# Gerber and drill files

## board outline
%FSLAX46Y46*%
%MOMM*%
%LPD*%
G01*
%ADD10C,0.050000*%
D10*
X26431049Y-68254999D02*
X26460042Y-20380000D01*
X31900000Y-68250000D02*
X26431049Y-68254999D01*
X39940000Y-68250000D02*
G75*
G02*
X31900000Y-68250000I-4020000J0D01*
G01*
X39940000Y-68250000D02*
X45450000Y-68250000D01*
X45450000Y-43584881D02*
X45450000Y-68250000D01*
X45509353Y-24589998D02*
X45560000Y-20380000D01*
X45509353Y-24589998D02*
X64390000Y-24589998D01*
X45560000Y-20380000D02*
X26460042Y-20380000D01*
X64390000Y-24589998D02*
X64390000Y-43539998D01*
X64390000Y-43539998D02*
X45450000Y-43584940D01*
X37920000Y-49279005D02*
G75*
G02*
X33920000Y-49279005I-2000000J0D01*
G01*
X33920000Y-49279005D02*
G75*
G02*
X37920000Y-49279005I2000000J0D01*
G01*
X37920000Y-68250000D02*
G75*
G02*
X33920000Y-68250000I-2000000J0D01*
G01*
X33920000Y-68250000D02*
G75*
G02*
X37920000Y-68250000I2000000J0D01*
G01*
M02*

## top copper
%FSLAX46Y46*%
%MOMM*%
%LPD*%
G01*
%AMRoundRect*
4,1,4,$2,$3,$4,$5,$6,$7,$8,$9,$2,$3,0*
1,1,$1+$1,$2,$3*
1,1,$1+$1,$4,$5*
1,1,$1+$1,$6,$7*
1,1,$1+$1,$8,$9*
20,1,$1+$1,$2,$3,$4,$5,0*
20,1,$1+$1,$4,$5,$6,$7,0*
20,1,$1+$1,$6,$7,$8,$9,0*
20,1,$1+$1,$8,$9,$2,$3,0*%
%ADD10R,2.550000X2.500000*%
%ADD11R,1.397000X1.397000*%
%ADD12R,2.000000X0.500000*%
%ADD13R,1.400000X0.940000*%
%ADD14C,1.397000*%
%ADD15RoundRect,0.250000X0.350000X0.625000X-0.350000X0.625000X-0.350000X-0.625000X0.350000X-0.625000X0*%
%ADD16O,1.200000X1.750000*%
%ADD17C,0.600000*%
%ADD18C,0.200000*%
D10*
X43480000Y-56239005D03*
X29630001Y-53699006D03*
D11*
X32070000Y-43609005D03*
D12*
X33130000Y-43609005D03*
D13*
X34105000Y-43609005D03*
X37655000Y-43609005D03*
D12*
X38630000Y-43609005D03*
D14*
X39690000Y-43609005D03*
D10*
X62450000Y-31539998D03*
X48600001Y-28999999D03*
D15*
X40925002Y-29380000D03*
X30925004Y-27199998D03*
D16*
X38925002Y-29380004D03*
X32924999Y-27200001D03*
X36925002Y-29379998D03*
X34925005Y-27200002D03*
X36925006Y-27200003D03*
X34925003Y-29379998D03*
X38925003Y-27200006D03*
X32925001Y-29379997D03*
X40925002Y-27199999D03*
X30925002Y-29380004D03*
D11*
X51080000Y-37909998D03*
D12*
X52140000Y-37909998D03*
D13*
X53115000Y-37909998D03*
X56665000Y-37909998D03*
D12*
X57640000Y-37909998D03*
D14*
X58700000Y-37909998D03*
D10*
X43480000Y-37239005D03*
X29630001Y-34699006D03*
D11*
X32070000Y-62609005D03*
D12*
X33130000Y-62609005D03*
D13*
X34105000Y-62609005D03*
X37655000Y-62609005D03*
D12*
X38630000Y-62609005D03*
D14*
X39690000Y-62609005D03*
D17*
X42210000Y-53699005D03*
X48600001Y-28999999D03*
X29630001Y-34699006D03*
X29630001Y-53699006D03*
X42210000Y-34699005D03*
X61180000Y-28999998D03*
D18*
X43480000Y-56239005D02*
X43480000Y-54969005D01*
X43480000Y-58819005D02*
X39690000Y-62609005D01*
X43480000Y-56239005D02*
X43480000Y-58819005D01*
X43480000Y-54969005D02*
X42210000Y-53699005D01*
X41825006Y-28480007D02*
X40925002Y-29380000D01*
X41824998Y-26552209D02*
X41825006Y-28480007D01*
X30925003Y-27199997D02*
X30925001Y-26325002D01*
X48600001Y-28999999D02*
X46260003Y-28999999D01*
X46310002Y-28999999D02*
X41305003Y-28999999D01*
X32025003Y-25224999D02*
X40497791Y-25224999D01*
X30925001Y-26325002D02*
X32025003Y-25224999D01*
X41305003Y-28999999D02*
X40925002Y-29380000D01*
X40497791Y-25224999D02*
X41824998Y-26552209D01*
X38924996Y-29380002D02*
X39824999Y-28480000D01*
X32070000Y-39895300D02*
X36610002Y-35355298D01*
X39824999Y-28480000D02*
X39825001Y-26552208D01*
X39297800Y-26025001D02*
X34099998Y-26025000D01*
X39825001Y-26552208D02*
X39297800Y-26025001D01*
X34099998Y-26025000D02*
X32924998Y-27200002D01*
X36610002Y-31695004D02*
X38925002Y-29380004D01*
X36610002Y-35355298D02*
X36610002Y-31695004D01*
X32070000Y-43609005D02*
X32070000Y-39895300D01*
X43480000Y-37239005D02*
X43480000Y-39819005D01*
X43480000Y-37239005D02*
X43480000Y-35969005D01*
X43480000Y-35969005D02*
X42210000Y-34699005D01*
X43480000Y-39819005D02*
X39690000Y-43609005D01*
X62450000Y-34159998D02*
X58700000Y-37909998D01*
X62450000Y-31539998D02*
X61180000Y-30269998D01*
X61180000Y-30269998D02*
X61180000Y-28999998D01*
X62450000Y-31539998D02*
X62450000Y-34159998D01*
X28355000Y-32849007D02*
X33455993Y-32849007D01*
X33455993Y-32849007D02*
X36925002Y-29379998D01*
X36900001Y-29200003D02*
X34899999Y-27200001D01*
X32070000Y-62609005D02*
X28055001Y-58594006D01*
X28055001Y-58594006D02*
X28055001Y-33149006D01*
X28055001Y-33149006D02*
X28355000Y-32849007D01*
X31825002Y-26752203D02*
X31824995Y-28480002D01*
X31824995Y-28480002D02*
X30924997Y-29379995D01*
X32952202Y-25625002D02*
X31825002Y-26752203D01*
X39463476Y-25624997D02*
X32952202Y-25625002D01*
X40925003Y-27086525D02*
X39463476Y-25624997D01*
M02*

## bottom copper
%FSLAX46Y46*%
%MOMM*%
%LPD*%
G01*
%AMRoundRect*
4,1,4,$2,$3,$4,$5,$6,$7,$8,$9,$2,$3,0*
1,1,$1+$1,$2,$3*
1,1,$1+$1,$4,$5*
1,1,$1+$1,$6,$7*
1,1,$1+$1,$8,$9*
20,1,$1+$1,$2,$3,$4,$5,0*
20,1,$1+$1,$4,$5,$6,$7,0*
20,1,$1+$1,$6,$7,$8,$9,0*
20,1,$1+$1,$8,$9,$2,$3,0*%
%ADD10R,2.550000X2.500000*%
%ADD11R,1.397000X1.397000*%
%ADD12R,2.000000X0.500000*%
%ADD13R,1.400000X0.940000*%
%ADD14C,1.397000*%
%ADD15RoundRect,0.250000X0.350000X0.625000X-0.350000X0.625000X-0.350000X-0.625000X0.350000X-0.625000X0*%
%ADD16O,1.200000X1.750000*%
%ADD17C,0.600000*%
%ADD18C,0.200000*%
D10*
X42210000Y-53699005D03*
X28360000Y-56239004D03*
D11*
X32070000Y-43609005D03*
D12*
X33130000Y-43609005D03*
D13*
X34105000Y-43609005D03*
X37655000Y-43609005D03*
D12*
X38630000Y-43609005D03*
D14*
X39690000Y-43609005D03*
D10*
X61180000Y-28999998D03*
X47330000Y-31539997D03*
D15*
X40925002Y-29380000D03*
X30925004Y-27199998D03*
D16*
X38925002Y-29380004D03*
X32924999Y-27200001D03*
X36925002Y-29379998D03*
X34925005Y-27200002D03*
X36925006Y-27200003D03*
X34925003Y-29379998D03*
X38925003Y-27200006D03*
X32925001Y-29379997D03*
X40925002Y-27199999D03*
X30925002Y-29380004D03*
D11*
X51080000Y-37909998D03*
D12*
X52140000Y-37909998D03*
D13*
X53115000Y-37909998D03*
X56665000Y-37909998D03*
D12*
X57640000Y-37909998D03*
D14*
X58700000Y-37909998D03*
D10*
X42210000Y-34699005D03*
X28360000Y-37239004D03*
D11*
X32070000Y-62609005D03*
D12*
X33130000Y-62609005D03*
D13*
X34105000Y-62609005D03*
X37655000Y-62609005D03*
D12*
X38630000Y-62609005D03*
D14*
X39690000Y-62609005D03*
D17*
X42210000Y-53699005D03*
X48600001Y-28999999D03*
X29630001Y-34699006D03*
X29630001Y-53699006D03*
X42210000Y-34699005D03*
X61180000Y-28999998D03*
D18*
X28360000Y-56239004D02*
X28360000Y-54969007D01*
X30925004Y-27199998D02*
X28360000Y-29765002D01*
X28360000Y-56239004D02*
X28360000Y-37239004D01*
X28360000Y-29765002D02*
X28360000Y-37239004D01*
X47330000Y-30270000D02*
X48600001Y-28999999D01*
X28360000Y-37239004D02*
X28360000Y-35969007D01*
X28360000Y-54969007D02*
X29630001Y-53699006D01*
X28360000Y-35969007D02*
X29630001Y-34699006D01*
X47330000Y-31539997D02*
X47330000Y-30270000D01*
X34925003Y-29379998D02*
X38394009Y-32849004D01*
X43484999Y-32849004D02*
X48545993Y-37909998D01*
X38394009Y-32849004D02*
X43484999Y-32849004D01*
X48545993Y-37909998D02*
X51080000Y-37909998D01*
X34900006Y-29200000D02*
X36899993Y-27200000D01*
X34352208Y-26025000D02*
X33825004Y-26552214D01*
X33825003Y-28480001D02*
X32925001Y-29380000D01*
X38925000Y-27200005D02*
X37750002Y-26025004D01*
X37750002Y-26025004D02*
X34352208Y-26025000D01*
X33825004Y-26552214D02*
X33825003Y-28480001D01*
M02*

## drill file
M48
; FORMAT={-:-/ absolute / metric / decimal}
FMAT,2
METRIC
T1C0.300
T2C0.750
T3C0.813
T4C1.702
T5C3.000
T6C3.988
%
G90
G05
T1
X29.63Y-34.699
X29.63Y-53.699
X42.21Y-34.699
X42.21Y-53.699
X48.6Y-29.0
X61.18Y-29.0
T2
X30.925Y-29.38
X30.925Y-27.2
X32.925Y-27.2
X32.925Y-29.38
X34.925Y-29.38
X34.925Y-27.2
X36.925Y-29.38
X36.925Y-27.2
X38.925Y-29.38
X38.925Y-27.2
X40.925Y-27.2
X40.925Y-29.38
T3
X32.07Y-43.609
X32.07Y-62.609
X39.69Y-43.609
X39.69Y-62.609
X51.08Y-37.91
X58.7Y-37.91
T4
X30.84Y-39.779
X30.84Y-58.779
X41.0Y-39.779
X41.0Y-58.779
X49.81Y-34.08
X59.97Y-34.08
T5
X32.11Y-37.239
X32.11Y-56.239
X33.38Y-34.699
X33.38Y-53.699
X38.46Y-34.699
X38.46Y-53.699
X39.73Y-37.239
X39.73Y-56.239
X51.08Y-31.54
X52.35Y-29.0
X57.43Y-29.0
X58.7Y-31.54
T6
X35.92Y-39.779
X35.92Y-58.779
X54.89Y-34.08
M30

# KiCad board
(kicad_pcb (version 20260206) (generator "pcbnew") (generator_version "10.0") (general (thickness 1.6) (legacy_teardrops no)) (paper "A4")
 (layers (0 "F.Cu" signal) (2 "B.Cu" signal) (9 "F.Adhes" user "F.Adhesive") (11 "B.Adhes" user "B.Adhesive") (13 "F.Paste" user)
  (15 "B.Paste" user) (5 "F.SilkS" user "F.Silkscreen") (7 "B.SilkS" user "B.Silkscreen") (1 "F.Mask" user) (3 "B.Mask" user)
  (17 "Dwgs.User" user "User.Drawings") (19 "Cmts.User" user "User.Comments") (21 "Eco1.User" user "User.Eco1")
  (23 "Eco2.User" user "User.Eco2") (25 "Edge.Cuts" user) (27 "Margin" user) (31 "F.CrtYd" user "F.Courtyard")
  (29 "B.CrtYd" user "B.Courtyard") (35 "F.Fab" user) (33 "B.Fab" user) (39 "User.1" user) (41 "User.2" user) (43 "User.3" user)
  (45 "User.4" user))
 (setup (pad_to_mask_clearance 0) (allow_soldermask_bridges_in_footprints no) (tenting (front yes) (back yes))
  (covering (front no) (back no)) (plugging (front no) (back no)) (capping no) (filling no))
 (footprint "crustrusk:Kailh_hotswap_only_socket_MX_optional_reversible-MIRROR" (layer "F.Cu") (at 35.92 58.779005)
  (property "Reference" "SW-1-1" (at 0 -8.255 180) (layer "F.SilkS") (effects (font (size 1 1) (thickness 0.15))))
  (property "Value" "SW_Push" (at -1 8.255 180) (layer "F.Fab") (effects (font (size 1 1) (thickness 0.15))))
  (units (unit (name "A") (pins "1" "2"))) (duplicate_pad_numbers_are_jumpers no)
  (pad "" np_thru_hole circle (at -5.08 0) (size 1.7018 1.7018) (drill 1.7018) (layers "*.Cu" "*.Mask"))
  (pad "" np_thru_hole circle (at -3.81 -2.54 180) (size 3 3) (drill 3) (layers "*.Cu" "*.Mask"))
  (pad "" np_thru_hole circle (at -2.54 -5.079998) (size 3 3) (drill 3) (layers "*.Cu" "*.Mask"))
  (pad "" np_thru_hole circle (at 0 0) (size 3.9878 3.9878) (drill 3.9878) (layers "*.Cu" "*.Mask"))
  (pad "" np_thru_hole circle (at 2.540002 -5.080001 180) (size 3 3) (drill 3) (layers "*.Cu" "*.Mask"))
  (pad "" np_thru_hole circle (at 3.81 -2.54) (size 3 3) (drill 3) (layers "*.Cu" "*.Mask"))
  (pad "" np_thru_hole circle (at 5.08 0) (size 1.7018 1.7018) (drill 1.7018) (layers "*.Cu" "*.Mask"))
  (pad "1" smd rect (at 6.29 -5.08 180) (size 2.55 2.5) (layers "B.Cu" "B.Mask" "B.Paste") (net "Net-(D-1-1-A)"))
  (pad "1" smd rect (at 7.56 -2.54) (size 2.55 2.5) (layers "F.Cu" "F.Mask" "F.Paste") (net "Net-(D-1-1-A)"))
  (pad "2" smd rect (at -7.56 -2.540001 180) (size 2.55 2.5) (layers "B.Cu" "B.Mask" "B.Paste") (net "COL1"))
  (pad "2" smd rect (at -6.289999 -5.079999) (size 2.55 2.5) (layers "F.Cu" "F.Mask" "F.Paste") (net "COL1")))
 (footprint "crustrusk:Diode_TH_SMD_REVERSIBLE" (layer "F.Cu") (at 35.88 43.609005)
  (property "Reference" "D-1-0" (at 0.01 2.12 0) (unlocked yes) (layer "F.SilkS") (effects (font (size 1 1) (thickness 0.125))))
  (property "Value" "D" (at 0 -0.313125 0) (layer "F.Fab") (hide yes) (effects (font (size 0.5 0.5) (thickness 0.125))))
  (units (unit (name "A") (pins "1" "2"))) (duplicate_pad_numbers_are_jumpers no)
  (pad "1" thru_hole rect (at -3.81 0) (size 1.397 1.397) (drill 0.8128) (layers "*.Cu" "*.Mask") (remove_unused_layers no) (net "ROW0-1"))
  (pad "1" smd rect (at -2.75 0 180) (size 2 0.5) (layers "F.Cu") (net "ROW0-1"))
  (pad "1" smd rect (at -2.75 0) (size 2 0.5) (layers "B.Cu") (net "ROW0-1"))
  (pad "1" smd rect (at -1.775 0 180) (size 1.4 0.94) (layers "F.Cu" "F.Mask" "F.Paste") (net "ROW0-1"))
  (pad "1" smd rect (at -1.775 0) (size 1.4 0.94) (layers "B.Cu" "B.Mask" "B.Paste") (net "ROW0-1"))
  (pad "2" smd rect (at 1.775 0 180) (size 1.4 0.94) (layers "F.Cu" "F.Mask" "F.Paste") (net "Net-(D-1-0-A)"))
  (pad "2" smd rect (at 1.775 0) (size 1.4 0.94) (layers "B.Cu" "B.Mask" "B.Paste") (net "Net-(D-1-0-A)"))
  (pad "2" smd rect (at 2.75 0 180) (size 2 0.5) (layers "F.Cu") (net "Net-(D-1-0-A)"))
  (pad "2" smd rect (at 2.75 0) (size 2 0.5) (layers "B.Cu") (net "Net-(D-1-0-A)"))
  (pad "2" thru_hole circle (at 3.81 0) (size 1.397 1.397) (drill 0.8128) (layers "*.Cu" "*.Mask") (remove_unused_layers no)
   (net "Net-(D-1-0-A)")))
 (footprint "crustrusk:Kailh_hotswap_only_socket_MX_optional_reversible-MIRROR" (layer "F.Cu") (at 54.89 34.079998)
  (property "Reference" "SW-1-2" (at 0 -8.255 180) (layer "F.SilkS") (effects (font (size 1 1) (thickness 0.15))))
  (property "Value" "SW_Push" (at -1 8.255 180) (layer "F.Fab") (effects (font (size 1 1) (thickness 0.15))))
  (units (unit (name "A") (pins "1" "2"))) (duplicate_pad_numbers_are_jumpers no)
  (pad "" np_thru_hole circle (at -5.08 0) (size 1.7018 1.7018) (drill 1.7018) (layers "*.Cu" "*.Mask"))
  (pad "" np_thru_hole circle (at -3.81 -2.54 180) (size 3 3) (drill 3) (layers "*.Cu" "*.Mask"))
  (pad "" np_thru_hole circle (at -2.54 -5.079998) (size 3 3) (drill 3) (layers "*.Cu" "*.Mask"))
  (pad "" np_thru_hole circle (at 0 0) (size 3.9878 3.9878) (drill 3.9878) (layers "*.Cu" "*.Mask"))
  (pad "" np_thru_hole circle (at 2.540002 -5.080001 180) (size 3 3) (drill 3) (layers "*.Cu" "*.Mask"))
  (pad "" np_thru_hole circle (at 3.81 -2.54) (size 3 3) (drill 3) (layers "*.Cu" "*.Mask"))
  (pad "" np_thru_hole circle (at 5.08 0) (size 1.7018 1.7018) (drill 1.7018) (layers "*.Cu" "*.Mask"))
  (pad "1" smd rect (at 6.29 -5.08 180) (size 2.55 2.5) (layers "B.Cu" "B.Mask" "B.Paste") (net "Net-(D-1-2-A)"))
  (pad "1" smd rect (at 7.56 -2.54) (size 2.55 2.5) (layers "F.Cu" "F.Mask" "F.Paste") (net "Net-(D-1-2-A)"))
  (pad "2" smd rect (at -7.56 -2.540001 180) (size 2.55 2.5) (layers "B.Cu" "B.Mask" "B.Paste") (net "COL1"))
  (pad "2" smd rect (at -6.289999 -5.079999) (size 2.55 2.5) (layers "F.Cu" "F.Mask" "F.Paste") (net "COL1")))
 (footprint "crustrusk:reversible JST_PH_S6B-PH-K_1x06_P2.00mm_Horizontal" (layer "F.Cu") (at 40.925002 29.38 180)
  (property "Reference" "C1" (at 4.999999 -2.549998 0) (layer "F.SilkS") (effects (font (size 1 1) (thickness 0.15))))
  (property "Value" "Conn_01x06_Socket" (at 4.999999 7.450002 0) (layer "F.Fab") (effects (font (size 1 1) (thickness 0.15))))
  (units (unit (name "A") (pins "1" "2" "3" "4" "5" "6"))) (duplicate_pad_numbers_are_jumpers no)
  (pad "1" thru_hole roundrect (at 0 0 180) (size 1.2 1.75) (drill 0.75) (layers "*.Cu" "*.Mask") (remove_unused_layers no)
   (roundrect_rratio 0.208333) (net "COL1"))
  (pad "1" thru_hole roundrect (at 9.999998 2.180002 180) (size 1.2 1.75) (drill 0.75) (layers "*.Cu" "*.Mask") (remove_unused_layers no)
   (roundrect_rratio 0.208333) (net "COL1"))
  (pad "2" thru_hole oval (at 2 -0.000004 180) (size 1.2 1.75) (drill 0.75) (layers "*.Cu" "*.Mask") (remove_unused_layers no)
   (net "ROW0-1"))
  (pad "2" thru_hole oval (at 8.000003 2.179999 180) (size 1.2 1.75) (drill 0.75) (layers "*.Cu" "*.Mask") (remove_unused_layers no)
   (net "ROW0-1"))
  (pad "3" thru_hole oval (at 4 0.000002 180) (size 1.2 1.75) (drill 0.75) (layers "*.Cu" "*.Mask") (remove_unused_layers no) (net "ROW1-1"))
  (pad "3" thru_hole oval (at 5.999997 2.179998 180) (size 1.2 1.75) (drill 0.75) (layers "*.Cu" "*.Mask") (remove_unused_layers no)
   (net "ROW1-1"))
  (pad "4" thru_hole oval (at 3.999996 2.179997 180) (size 1.2 1.75) (drill 0.75) (layers "*.Cu" "*.Mask") (remove_unused_layers no)
   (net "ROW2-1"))
  (pad "4" thru_hole oval (at 5.999999 0.000002 180) (size 1.2 1.75) (drill 0.75) (layers "*.Cu" "*.Mask") (remove_unused_layers no)
   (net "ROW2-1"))
  (pad "5" thru_hole oval (at 1.999999 2.179994 180) (size 1.2 1.75) (drill 0.75) (layers "*.Cu" "*.Mask") (remove_unused_layers no)
   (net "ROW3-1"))
  (pad "5" thru_hole oval (at 8.000001 0.000003 180) (size 1.2 1.75) (drill 0.75) (layers "*.Cu" "*.Mask") (remove_unused_layers no)
   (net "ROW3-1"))
  (pad "6" thru_hole oval (at 0 2.180001 180) (size 1.2 1.75) (drill 0.75) (layers "*.Cu" "*.Mask") (remove_unused_layers no) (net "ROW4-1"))
  (pad "6" thru_hole oval (at 10 -0.000004 180) (size 1.2 1.75) (drill 0.75) (layers "*.Cu" "*.Mask") (remove_unused_layers no)
   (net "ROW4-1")))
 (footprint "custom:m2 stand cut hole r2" (layer "F.Cu") (at 35.92 49.279005)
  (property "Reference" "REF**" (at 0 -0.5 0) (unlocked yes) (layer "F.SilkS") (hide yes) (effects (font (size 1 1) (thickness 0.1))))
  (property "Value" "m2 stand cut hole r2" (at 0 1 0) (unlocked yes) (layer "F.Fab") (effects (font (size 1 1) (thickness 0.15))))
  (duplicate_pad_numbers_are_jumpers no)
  (fp_circle (center 0 0) (end 2 0) (stroke (width 0.05) (type default)) (fill no) (layer "Edge.Cuts")))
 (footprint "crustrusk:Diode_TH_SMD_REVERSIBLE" (layer "F.Cu") (at 54.89 37.909998)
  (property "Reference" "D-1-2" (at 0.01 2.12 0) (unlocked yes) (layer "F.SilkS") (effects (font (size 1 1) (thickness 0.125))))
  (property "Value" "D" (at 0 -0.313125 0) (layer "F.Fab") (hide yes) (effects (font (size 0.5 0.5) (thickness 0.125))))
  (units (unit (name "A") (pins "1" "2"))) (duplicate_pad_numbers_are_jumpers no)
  (pad "1" thru_hole rect (at -3.81 0) (size 1.397 1.397) (drill 0.8128) (layers "*.Cu" "*.Mask") (remove_unused_layers no) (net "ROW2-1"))
  (pad "1" smd rect (at -2.75 0 180) (size 2 0.5) (layers "F.Cu") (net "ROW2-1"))
  (pad "1" smd rect (at -2.75 0) (size 2 0.5) (layers "B.Cu") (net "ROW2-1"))
  (pad "1" smd rect (at -1.775 0 180) (size 1.4 0.94) (layers "F.Cu" "F.Mask" "F.Paste") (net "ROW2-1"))
  (pad "1" smd rect (at -1.775 0) (size 1.4 0.94) (layers "B.Cu" "B.Mask" "B.Paste") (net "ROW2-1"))
  (pad "2" smd rect (at 1.775 0 180) (size 1.4 0.94) (layers "F.Cu" "F.Mask" "F.Paste") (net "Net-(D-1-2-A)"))
  (pad "2" smd rect (at 1.775 0) (size 1.4 0.94) (layers "B.Cu" "B.Mask" "B.Paste") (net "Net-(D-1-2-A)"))
  (pad "2" smd rect (at 2.75 0 180) (size 2 0.5) (layers "F.Cu") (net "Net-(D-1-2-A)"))
  (pad "2" smd rect (at 2.75 0) (size 2 0.5) (layers "B.Cu") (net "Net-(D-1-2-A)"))
  (pad "2" thru_hole circle (at 3.81 0) (size 1.397 1.397) (drill 0.8128) (layers "*.Cu" "*.Mask") (remove_unused_layers no)
   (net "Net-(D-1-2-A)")))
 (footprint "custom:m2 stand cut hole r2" (layer "F.Cu") (at 35.92 68.25)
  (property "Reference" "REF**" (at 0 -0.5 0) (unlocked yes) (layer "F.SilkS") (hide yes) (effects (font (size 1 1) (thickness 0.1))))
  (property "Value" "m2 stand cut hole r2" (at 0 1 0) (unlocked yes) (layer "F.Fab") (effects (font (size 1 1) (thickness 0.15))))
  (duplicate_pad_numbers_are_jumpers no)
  (fp_circle (center 0 0) (end 2 0) (stroke (width 0.05) (type default)) (fill no) (layer "Edge.Cuts")))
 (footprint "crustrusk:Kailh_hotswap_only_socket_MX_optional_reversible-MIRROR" (layer "F.Cu") (at 35.92 39.779005)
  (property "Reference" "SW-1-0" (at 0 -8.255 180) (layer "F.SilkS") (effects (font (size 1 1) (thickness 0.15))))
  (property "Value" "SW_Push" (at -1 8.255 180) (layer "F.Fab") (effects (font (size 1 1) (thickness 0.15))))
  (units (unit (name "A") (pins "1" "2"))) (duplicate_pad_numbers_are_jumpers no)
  (pad "" np_thru_hole circle (at -5.08 0) (size 1.7018 1.7018) (drill 1.7018) (layers "*.Cu" "*.Mask"))
  (pad "" np_thru_hole circle (at -3.81 -2.54 180) (size 3 3) (drill 3) (layers "*.Cu" "*.Mask"))
  (pad "" np_thru_hole circle (at -2.54 -5.079998) (size 3 3) (drill 3) (layers "*.Cu" "*.Mask"))
  (pad "" np_thru_hole circle (at 0 0) (size 3.9878 3.9878) (drill 3.9878) (layers "*.Cu" "*.Mask"))
  (pad "" np_thru_hole circle (at 2.540002 -5.080001 180) (size 3 3) (drill 3) (layers "*.Cu" "*.Mask"))
  (pad "" np_thru_hole circle (at 3.81 -2.54) (size 3 3) (drill 3) (layers "*.Cu" "*.Mask"))
  (pad "" np_thru_hole circle (at 5.08 0) (size 1.7018 1.7018) (drill 1.7018) (layers "*.Cu" "*.Mask"))
  (pad "1" smd rect (at 6.29 -5.08 180) (size 2.55 2.5) (layers "B.Cu" "B.Mask" "B.Paste") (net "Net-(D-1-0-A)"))
  (pad "1" smd rect (at 7.56 -2.54) (size 2.55 2.5) (layers "F.Cu" "F.Mask" "F.Paste") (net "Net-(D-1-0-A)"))
  (pad "2" smd rect (at -7.56 -2.540001 180) (size 2.55 2.5) (layers "B.Cu" "B.Mask" "B.Paste") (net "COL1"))
  (pad "2" smd rect (at -6.289999 -5.079999) (size 2.55 2.5) (layers "F.Cu" "F.Mask" "F.Paste") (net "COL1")))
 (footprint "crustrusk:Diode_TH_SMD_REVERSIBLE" (layer "F.Cu") (at 35.88 62.609005)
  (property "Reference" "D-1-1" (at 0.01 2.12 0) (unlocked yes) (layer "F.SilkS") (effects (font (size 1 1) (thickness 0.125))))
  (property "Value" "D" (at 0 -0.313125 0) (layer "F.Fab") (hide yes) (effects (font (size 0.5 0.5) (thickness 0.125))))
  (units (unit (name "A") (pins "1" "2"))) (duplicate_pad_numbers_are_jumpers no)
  (pad "1" thru_hole rect (at -3.81 0) (size 1.397 1.397) (drill 0.8128) (layers "*.Cu" "*.Mask") (remove_unused_layers no) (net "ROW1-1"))
  (pad "1" smd rect (at -2.75 0 180) (size 2 0.5) (layers "F.Cu") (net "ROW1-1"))
  (pad "1" smd rect (at -2.75 0) (size 2 0.5) (layers "B.Cu") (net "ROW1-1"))
  (pad "1" smd rect (at -1.775 0 180) (size 1.4 0.94) (layers "F.Cu" "F.Mask" "F.Paste") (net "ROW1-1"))
  (pad "1" smd rect (at -1.775 0) (size 1.4 0.94) (layers "B.Cu" "B.Mask" "B.Paste") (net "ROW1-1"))
  (pad "2" smd rect (at 1.775 0 180) (size 1.4 0.94) (layers "F.Cu" "F.Mask" "F.Paste") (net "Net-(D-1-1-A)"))
  (pad "2" smd rect (at 1.775 0) (size 1.4 0.94) (layers "B.Cu" "B.Mask" "B.Paste") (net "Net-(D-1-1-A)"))
  (pad "2" smd rect (at 2.75 0 180) (size 2 0.5) (layers "F.Cu") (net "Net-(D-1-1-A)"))
  (pad "2" smd rect (at 2.75 0) (size 2 0.5) (layers "B.Cu") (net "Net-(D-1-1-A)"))
  (pad "2" thru_hole circle (at 3.81 0) (size 1.397 1.397) (drill 0.8128) (layers "*.Cu" "*.Mask") (remove_unused_layers no)
   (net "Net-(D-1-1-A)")))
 (gr_line (start 26.431049 68.254999) (end 26.460042 20.38) (stroke (width 0.05) (type default)) (layer "Edge.Cuts"))
 (gr_line (start 31.9 68.25) (end 26.431049 68.254999) (stroke (width 0.05) (type default)) (layer "Edge.Cuts"))
 (gr_arc (start 39.94 68.25) (mid 35.92 72.27) (end 31.9 68.25) (stroke (width 0.05) (type default)) (layer "Edge.Cuts"))
 (gr_line (start 39.94 68.25) (end 45.45 68.25) (stroke (width 0.05) (type default)) (layer "Edge.Cuts"))
 (gr_line (start 45.45 43.584881) (end 45.45 68.25) (stroke (width 0.05) (type default)) (layer "Edge.Cuts"))
 (gr_line (start 45.509353 24.589998) (end 45.56 20.38) (stroke (width 0.05) (type default)) (layer "Edge.Cuts"))
 (gr_line (start 45.509353 24.589998) (end 64.39 24.589998) (stroke (width 0.05) (type default)) (layer "Edge.Cuts"))
 (gr_line (start 45.56 20.38) (end 26.460042 20.38) (stroke (width 0.05) (type default)) (layer "Edge.Cuts"))
 (gr_line (start 64.39 24.589998) (end 64.39 43.539998) (stroke (width 0.05) (type default)) (layer "Edge.Cuts"))
 (gr_line (start 64.39 43.539998) (end 45.45 43.58494) (stroke (width 0.05) (type default)) (layer "Edge.Cuts"))
 (segment (start 43.48 56.239005) (end 43.48 54.969005) (width 0.2) (layer "F.Cu") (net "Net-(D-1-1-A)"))
 (segment (start 43.48 58.819005) (end 39.69 62.609005) (width 0.2) (layer "F.Cu") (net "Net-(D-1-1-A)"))
 (segment (start 43.48 56.239005) (end 43.48 58.819005) (width 0.2) (layer "F.Cu") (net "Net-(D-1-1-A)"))
 (segment (start 43.48 54.969005) (end 42.21 53.699005) (width 0.2) (layer "F.Cu") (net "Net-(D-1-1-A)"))
 (via (at 42.21 53.699005) (size 0.6) (drill 0.3) (layers "F.Cu" "B.Cu") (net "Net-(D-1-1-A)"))
 (segment (start 41.825006 28.480007) (end 40.925002 29.38) (width 0.2) (layer "F.Cu") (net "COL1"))
 (segment (start 41.824998 26.552209) (end 41.825006 28.480007) (width 0.2) (layer "F.Cu") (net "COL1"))
 (segment (start 30.925003 27.199997) (end 30.925001 26.325002) (width 0.2) (layer "F.Cu") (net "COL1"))
 (segment (start 48.600001 28.999999) (end 46.260003 28.999999) (width 0.2) (layer "F.Cu") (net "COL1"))
 (segment (start 46.310002 28.999999) (end 41.305003 28.999999) (width 0.2) (layer "F.Cu") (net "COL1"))
 (segment (start 32.025003 25.224999) (end 40.497791 25.224999) (width 0.2) (layer "F.Cu") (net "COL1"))
 (segment (start 30.925001 26.325002) (end 32.025003 25.224999) (width 0.2) (layer "F.Cu") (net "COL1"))
 (segment (start 41.305003 28.999999) (end 40.925002 29.38) (width 0.2) (layer "F.Cu") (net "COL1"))
 (segment (start 40.497791 25.224999) (end 41.824998 26.552209) (width 0.2) (layer "F.Cu") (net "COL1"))
 (via (at 48.600001 28.999999) (size 0.6) (drill 0.3) (layers "F.Cu" "B.Cu") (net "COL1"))
 (via (at 29.630001 34.699006) (size 0.6) (drill 0.3) (layers "F.Cu" "B.Cu") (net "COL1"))
 (via (at 29.630001 53.699006) (size 0.6) (drill 0.3) (layers "F.Cu" "B.Cu") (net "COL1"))
 (segment (start 28.36 56.239004) (end 28.36 54.969007) (width 0.2) (layer "B.Cu") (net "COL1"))
 (segment (start 30.925004 27.199998) (end 28.36 29.765002) (width 0.2) (layer "B.Cu") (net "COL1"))
 (segment (start 28.36 56.239004) (end 28.36 37.239004) (width 0.2) (layer "B.Cu") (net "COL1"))
 (segment (start 28.36 29.765002) (end 28.36 37.239004) (width 0.2) (layer "B.Cu") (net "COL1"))
 (segment (start 47.33 30.27) (end 48.600001 28.999999) (width 0.2) (layer "B.Cu") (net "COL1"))
 (segment (start 28.36 37.239004) (end 28.36 35.969007) (width 0.2) (layer "B.Cu") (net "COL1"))
 (segment (start 28.36 54.969007) (end 29.630001 53.699006) (width 0.2) (layer "B.Cu") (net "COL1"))
 (segment (start 28.36 35.969007) (end 29.630001 34.699006) (width 0.2) (layer "B.Cu") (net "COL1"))
 (segment (start 47.33 31.539997) (end 47.33 30.27) (width 0.2) (layer "B.Cu") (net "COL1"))
 (segment (start 38.924996 29.380002) (end 39.824999 28.48) (width 0.2) (layer "F.Cu") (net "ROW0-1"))
 (segment (start 32.07 39.8953) (end 36.610002 35.355298) (width 0.2) (layer "F.Cu") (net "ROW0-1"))
 (segment (start 39.824999 28.48) (end 39.825001 26.552208) (width 0.2) (layer "F.Cu") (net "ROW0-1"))
 (segment (start 39.2978 26.025001) (end 34.099998 26.025) (width 0.2) (layer "F.Cu") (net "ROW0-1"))
 (segment (start 39.825001 26.552208) (end 39.2978 26.025001) (width 0.2) (layer "F.Cu") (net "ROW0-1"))
 (segment (start 34.099998 26.025) (end 32.924998 27.200002) (width 0.2) (layer "F.Cu") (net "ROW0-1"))
 (segment (start 36.610002 31.695004) (end 38.925002 29.380004) (width 0.2) (layer "F.Cu") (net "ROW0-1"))
 (segment (start 36.610002 35.355298) (end 36.610002 31.695004) (width 0.2) (layer "F.Cu") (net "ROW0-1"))
 (segment (start 32.07 43.609005) (end 32.07 39.8953) (width 0.2) (layer "F.Cu") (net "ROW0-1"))
 (segment (start 43.48 37.239005) (end 43.48 39.819005) (width 0.2) (layer "F.Cu") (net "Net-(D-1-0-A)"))
 (segment (start 43.48 37.239005) (end 43.48 35.969005) (width 0.2) (layer "F.Cu") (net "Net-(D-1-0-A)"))
 (segment (start 43.48 35.969005) (end 42.21 34.699005) (width 0.2) (layer "F.Cu") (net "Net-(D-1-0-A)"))
 (segment (start 43.48 39.819005) (end 39.69 43.609005) (width 0.2) (layer "F.Cu") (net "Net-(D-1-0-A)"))
 (via (at 42.21 34.699005) (size 0.6) (drill 0.3) (layers "F.Cu" "B.Cu") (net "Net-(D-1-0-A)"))
 (segment (start 62.45 34.159998) (end 58.7 37.909998) (width 0.2) (layer "F.Cu") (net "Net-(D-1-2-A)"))
 (segment (start 62.45 31.539998) (end 61.18 30.269998) (width 0.2) (layer "F.Cu") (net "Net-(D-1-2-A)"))
 (segment (start 61.18 30.269998) (end 61.18 28.999998) (width 0.2) (layer "F.Cu") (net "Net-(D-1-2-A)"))
 (segment (start 62.45 31.539998) (end 62.45 34.159998) (width 0.2) (layer "F.Cu") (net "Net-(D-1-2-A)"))
 (via (at 61.18 28.999998) (size 0.6) (drill 0.3) (layers "F.Cu" "B.Cu") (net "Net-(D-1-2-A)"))
 (segment (start 28.355 32.849007) (end 33.455993 32.849007) (width 0.2) (layer "F.Cu") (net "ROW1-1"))
 (segment (start 33.455993 32.849007) (end 36.925002 29.379998) (width 0.2) (layer "F.Cu") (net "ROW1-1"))
 (segment (start 36.900001 29.200003) (end 34.899999 27.200001) (width 0.2) (layer "F.Cu") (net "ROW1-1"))
 (segment (start 32.07 62.609005) (end 28.055001 58.594006) (width 0.2) (layer "F.Cu") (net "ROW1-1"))
 (segment (start 28.055001 58.594006) (end 28.055001 33.149006) (width 0.2) (layer "F.Cu") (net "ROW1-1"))
 (segment (start 28.055001 33.149006) (end 28.355 32.849007) (width 0.2) (layer "F.Cu") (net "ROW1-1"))
 (segment (start 34.925003 29.379998) (end 38.394009 32.849004) (width 0.2) (layer "B.Cu") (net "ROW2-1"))
 (segment (start 43.484999 32.849004) (end 48.545993 37.909998) (width 0.2) (layer "B.Cu") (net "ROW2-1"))
 (segment (start 38.394009 32.849004) (end 43.484999 32.849004) (width 0.2) (layer "B.Cu") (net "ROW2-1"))
 (segment (start 48.545993 37.909998) (end 51.08 37.909998) (width 0.2) (layer "B.Cu") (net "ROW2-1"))
 (segment (start 34.900006 29.2) (end 36.899993 27.2) (width 0.2) (layer "B.Cu") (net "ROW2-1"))
 (segment (start 34.352208 26.025) (end 33.825004 26.552214) (width 0.2) (layer "B.Cu") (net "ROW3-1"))
 (segment (start 33.825003 28.480001) (end 32.925001 29.38) (width 0.2) (layer "B.Cu") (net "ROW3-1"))
 (segment (start 38.925 27.200005) (end 37.750002 26.025004) (width 0.2) (layer "B.Cu") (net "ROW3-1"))
 (segment (start 37.750002 26.025004) (end 34.352208 26.025) (width 0.2) (layer "B.Cu") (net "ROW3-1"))
 (segment (start 33.825004 26.552214) (end 33.825003 28.480001) (width 0.2) (layer "B.Cu") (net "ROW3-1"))
 (segment (start 31.825002 26.752203) (end 31.824995 28.480002) (width 0.2) (layer "F.Cu") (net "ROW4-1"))
 (segment (start 31.824995 28.480002) (end 30.924997 29.379995) (width 0.2) (layer "F.Cu") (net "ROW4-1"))
 (segment (start 32.952202 25.625002) (end 31.825002 26.752203) (width 0.2) (layer "F.Cu") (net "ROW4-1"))
 (segment (start 39.463476 25.624997) (end 32.952202 25.625002) (width 0.2) (layer "F.Cu") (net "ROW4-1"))
 (segment (start 40.925003 27.086525) (end 39.463476 25.624997) (width 0.2) (layer "F.Cu") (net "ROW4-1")))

